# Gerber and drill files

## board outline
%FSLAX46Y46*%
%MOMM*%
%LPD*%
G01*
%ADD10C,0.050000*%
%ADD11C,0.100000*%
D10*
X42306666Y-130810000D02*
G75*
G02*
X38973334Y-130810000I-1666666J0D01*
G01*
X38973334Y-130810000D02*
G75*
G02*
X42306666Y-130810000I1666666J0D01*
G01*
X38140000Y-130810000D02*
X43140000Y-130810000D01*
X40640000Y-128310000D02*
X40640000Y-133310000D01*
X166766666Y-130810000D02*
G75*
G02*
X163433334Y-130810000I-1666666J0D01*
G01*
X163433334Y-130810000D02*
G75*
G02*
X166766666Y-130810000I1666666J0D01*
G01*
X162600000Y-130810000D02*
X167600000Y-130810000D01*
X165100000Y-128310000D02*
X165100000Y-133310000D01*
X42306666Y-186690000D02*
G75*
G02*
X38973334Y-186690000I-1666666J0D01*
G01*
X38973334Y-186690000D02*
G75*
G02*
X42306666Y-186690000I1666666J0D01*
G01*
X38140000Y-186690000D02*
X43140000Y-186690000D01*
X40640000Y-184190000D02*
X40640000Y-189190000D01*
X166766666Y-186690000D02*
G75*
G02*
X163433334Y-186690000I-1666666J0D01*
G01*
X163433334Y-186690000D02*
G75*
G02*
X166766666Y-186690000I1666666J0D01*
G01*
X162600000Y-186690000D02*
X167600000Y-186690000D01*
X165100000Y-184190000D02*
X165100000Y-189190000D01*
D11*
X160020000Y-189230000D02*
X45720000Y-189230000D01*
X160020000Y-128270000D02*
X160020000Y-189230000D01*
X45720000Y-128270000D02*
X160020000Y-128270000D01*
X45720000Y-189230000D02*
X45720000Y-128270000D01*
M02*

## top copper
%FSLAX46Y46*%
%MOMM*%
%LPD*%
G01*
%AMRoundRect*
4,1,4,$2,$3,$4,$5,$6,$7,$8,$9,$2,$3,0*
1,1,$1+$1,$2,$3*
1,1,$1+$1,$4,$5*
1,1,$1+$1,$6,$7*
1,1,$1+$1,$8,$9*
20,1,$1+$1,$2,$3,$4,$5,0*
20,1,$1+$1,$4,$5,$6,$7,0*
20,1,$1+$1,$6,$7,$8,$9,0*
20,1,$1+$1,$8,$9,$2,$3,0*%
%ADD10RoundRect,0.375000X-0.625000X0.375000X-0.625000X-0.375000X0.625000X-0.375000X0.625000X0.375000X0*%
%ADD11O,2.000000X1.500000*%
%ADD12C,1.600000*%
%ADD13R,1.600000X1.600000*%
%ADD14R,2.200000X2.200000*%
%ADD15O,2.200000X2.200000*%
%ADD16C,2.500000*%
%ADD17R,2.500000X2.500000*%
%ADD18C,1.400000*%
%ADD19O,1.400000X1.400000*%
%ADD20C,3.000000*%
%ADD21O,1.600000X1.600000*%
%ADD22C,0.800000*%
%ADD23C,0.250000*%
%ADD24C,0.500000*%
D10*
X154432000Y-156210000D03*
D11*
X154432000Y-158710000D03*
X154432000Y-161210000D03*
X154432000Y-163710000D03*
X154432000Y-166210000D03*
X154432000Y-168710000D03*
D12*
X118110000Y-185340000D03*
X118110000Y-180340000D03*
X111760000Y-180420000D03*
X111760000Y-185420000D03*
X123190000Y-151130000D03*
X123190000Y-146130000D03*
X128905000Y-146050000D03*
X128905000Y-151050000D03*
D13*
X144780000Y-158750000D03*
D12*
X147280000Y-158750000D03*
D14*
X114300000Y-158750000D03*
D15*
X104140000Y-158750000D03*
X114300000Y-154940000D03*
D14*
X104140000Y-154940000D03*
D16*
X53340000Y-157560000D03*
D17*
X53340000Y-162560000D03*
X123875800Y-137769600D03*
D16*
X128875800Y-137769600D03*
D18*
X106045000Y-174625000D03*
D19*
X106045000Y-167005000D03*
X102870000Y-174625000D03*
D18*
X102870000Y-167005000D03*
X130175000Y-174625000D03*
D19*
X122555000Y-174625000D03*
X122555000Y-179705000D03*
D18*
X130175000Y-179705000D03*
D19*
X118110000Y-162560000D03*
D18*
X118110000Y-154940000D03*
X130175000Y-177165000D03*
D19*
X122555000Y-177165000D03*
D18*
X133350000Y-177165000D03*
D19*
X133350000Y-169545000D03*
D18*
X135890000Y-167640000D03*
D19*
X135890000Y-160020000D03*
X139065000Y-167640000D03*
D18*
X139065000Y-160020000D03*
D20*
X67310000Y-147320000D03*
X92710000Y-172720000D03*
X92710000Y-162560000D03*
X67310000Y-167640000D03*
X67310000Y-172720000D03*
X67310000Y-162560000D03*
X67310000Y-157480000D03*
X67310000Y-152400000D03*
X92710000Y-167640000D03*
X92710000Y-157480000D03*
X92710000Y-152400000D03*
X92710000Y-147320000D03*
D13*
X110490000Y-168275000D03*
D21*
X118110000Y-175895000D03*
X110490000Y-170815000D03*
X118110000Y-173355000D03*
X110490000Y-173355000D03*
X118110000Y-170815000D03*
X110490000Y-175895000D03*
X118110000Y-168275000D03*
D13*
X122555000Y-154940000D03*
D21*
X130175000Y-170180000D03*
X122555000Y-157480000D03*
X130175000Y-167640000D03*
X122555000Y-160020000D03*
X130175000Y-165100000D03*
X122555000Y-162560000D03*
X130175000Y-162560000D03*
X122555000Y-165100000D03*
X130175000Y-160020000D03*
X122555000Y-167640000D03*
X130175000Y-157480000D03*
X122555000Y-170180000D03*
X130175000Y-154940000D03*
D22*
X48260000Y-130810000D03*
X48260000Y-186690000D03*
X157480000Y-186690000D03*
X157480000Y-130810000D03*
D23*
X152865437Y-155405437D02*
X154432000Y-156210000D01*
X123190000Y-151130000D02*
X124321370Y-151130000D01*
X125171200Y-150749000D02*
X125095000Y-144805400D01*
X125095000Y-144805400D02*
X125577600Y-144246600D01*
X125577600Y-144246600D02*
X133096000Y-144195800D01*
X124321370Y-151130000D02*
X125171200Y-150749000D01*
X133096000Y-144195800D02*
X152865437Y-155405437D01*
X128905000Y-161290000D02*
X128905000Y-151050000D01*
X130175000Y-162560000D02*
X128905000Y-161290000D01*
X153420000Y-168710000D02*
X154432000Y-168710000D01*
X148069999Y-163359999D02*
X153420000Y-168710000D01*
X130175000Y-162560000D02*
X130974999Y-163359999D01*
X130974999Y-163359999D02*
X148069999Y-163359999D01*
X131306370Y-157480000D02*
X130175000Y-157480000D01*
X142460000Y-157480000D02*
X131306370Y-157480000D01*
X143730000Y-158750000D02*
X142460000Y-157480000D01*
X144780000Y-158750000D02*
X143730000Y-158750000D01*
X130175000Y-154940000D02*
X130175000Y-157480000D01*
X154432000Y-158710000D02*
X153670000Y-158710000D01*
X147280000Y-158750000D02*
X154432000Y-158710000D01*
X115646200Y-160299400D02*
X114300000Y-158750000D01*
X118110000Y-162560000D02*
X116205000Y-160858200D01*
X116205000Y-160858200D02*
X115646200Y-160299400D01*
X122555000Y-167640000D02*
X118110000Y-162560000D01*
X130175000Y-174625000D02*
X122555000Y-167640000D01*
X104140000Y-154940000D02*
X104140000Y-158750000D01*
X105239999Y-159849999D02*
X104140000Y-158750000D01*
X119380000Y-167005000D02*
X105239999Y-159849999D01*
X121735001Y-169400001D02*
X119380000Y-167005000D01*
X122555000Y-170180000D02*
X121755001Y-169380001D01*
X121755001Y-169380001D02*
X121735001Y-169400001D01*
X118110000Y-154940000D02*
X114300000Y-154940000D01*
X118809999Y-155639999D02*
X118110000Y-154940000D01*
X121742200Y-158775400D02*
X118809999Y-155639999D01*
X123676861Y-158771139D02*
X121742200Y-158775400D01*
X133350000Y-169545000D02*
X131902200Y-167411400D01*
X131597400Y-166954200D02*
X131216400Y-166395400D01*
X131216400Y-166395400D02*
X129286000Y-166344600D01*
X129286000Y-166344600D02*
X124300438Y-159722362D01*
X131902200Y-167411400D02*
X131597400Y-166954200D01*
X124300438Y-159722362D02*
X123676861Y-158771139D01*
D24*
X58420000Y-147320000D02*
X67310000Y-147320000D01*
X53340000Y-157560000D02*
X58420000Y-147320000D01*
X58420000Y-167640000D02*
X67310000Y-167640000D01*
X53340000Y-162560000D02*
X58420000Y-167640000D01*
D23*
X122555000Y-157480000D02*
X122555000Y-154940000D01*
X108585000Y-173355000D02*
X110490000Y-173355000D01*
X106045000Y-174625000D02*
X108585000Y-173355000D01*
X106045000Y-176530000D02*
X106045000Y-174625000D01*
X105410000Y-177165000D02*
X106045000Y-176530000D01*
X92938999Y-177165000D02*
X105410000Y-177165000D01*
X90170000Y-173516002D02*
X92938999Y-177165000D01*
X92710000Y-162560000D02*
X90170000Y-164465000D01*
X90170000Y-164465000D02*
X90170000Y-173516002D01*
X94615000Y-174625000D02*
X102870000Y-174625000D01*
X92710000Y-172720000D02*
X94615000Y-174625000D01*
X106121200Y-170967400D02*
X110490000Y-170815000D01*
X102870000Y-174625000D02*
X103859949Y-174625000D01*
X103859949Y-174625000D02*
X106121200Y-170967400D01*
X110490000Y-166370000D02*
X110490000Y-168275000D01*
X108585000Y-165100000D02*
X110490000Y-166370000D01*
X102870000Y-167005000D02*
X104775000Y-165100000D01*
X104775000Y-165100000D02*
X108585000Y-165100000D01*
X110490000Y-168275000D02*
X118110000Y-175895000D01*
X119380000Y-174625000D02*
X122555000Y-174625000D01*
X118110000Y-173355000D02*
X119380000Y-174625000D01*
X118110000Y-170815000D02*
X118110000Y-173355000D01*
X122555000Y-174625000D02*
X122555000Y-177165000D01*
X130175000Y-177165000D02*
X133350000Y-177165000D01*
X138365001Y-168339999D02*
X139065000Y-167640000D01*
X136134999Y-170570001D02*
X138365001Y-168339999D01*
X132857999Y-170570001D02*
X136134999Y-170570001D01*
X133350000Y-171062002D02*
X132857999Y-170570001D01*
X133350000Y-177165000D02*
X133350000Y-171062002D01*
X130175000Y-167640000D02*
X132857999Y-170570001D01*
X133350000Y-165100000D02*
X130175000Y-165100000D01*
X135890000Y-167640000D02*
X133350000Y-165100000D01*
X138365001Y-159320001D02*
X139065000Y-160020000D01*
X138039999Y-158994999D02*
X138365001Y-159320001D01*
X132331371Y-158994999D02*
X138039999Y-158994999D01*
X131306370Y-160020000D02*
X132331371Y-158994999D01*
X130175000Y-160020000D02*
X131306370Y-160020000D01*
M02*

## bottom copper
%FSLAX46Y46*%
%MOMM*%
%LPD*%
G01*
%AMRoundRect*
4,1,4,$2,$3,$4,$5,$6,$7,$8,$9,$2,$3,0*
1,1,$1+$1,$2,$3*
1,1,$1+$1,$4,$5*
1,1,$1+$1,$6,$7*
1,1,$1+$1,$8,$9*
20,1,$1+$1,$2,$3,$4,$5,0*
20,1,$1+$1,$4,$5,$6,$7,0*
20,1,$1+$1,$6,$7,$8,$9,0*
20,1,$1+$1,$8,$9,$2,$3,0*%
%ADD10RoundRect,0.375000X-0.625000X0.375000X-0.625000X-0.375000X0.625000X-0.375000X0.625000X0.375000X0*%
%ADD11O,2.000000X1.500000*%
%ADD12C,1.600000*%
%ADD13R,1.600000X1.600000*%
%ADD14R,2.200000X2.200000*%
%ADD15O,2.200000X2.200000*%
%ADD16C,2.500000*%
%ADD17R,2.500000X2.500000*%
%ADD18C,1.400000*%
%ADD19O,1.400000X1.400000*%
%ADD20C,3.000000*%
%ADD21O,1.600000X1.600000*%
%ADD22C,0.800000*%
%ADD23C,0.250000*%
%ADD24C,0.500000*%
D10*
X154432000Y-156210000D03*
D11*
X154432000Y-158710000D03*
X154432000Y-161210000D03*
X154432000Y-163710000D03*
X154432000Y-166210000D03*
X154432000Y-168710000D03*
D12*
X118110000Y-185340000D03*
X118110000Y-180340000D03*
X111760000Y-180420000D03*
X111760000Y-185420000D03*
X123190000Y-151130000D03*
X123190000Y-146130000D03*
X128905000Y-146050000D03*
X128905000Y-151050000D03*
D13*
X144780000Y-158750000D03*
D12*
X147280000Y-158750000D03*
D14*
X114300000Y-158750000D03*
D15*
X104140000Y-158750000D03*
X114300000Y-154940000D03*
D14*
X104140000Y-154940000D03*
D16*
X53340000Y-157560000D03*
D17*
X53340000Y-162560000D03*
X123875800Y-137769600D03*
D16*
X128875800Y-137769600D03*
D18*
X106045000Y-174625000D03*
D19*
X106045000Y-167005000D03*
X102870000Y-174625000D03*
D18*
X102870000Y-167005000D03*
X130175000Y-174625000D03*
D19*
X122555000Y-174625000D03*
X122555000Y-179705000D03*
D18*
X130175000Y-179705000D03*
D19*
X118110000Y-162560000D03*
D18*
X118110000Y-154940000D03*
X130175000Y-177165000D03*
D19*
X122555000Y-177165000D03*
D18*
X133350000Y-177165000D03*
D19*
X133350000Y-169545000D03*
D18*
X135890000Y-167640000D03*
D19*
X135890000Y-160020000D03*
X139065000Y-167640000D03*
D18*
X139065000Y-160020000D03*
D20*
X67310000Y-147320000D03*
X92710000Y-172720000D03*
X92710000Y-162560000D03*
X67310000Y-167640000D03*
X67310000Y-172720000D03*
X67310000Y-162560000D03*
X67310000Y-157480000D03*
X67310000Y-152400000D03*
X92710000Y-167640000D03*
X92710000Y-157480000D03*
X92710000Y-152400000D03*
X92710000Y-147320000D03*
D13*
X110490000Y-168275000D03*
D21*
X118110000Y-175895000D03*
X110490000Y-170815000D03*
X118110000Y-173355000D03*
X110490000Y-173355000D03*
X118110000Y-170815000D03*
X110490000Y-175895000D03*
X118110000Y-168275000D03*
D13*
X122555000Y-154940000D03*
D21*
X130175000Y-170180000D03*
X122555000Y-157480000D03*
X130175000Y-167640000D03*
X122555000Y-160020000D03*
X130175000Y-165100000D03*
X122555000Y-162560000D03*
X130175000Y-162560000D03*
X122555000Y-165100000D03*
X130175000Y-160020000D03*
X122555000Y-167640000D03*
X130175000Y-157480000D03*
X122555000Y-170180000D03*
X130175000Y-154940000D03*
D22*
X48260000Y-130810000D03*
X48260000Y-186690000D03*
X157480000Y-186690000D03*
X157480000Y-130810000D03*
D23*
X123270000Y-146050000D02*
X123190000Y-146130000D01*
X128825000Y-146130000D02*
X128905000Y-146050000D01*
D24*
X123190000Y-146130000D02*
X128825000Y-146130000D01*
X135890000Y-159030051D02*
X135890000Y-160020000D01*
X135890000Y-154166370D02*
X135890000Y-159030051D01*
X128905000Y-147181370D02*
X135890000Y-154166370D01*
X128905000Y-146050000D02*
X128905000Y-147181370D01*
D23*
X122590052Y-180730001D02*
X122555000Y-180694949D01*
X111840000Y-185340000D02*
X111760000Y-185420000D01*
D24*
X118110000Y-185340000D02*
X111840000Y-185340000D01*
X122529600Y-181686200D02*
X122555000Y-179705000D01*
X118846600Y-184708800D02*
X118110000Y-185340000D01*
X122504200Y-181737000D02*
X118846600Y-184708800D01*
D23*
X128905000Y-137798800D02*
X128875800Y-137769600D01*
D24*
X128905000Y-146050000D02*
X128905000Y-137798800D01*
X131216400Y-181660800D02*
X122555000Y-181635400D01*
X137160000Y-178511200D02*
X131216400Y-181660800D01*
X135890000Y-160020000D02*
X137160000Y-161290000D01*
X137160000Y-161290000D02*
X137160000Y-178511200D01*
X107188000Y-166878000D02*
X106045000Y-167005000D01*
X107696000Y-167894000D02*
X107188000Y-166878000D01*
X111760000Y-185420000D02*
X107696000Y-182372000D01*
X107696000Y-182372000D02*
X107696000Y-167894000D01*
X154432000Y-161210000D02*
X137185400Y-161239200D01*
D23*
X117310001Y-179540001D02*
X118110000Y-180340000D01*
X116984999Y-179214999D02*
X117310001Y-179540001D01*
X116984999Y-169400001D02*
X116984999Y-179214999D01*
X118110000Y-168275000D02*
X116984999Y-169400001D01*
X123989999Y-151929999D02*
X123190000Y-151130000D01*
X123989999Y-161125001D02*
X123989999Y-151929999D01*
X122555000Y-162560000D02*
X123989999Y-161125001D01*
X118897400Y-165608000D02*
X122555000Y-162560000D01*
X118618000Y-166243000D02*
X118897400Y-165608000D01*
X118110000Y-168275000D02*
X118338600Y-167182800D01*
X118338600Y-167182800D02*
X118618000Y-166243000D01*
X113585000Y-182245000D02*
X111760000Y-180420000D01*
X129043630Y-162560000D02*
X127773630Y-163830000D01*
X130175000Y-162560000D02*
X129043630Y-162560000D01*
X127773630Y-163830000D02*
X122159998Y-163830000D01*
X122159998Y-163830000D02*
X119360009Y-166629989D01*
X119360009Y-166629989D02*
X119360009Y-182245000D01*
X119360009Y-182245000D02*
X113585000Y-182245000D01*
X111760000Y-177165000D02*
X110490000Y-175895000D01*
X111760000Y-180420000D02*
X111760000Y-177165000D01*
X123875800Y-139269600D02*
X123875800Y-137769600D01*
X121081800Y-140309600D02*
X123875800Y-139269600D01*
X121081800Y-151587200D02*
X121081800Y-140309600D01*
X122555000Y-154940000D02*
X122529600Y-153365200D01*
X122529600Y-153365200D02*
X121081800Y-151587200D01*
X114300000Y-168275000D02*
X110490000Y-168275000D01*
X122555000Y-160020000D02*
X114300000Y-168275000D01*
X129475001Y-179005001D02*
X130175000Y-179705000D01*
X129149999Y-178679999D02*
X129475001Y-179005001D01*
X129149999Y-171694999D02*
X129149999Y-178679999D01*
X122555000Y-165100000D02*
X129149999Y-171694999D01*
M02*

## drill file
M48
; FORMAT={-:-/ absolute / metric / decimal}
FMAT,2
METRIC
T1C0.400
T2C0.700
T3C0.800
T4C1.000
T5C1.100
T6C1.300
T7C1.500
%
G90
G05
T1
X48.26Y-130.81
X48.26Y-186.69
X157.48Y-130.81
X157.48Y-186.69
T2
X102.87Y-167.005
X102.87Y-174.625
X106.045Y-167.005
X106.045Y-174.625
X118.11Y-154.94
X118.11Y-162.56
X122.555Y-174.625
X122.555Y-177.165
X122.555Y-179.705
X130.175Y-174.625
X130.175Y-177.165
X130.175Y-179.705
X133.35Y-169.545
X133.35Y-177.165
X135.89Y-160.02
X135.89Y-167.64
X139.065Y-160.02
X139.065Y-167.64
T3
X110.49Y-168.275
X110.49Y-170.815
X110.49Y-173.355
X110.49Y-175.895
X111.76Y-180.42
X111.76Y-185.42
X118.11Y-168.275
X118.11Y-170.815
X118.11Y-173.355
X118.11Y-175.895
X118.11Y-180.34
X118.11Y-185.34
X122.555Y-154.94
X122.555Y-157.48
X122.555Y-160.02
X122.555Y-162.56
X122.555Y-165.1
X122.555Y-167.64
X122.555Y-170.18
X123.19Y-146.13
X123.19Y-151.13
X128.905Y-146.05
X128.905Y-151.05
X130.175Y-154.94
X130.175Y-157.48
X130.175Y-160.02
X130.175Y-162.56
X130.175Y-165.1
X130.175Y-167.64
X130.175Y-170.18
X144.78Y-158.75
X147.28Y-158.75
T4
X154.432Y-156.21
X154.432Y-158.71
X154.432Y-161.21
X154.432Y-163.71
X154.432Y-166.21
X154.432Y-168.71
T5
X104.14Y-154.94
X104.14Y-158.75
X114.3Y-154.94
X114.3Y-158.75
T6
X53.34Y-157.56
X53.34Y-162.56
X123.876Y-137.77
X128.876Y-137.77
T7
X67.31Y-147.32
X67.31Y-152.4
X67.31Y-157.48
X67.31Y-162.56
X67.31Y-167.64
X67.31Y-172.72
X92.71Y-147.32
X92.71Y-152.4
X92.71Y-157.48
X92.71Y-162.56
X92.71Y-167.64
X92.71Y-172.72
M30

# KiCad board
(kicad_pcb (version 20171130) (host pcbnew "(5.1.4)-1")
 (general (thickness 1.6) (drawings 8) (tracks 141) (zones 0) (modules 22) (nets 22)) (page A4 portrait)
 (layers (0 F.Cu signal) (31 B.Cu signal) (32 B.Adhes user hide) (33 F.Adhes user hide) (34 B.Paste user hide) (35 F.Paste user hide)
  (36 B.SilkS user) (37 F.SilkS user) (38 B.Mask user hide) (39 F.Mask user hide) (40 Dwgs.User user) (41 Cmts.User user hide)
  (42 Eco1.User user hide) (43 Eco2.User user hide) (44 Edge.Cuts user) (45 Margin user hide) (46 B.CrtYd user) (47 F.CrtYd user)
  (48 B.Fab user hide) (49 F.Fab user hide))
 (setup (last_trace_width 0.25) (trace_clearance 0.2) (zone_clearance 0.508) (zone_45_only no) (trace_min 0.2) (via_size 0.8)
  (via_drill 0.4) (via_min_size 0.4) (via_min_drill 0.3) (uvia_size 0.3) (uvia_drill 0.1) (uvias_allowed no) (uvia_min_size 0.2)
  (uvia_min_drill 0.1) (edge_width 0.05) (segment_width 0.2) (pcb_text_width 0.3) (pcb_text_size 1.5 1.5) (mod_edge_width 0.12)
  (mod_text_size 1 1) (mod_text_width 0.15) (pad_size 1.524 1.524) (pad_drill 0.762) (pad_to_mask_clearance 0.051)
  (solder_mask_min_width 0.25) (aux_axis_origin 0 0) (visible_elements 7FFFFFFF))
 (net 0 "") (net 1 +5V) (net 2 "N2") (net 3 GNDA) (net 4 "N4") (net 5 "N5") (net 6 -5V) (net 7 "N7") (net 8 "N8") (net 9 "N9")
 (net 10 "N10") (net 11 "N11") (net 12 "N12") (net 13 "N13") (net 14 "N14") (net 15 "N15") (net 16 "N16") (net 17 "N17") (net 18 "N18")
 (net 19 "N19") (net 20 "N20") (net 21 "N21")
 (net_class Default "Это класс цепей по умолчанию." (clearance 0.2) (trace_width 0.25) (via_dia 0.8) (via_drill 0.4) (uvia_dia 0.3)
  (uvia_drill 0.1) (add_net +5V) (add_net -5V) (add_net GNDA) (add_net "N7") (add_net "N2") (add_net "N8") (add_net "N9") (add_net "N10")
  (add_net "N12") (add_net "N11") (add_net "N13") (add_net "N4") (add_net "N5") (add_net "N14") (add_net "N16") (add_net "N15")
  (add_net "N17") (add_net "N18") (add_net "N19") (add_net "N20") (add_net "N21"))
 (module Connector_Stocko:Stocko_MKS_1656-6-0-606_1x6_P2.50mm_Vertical (layer F.Cu) (at 154.432 156.21 270)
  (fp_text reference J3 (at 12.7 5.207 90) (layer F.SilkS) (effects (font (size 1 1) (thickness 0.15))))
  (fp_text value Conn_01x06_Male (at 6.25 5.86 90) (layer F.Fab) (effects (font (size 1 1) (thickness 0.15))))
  (pad 1 thru_hole roundrect (at 0 0 270) (size 1.5 2) (drill 1) (layers *.Cu *.Mask) (roundrect_rratio 0.25) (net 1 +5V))
  (pad 2 thru_hole oval (at 2.5 0 270) (size 1.5 2) (drill 1) (layers *.Cu *.Mask) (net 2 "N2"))
  (pad 3 thru_hole oval (at 5 0 270) (size 1.5 2) (drill 1) (layers *.Cu *.Mask) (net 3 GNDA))
  (pad 4 thru_hole oval (at 7.5 0 270) (size 1.5 2) (drill 1) (layers *.Cu *.Mask) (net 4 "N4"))
  (pad 5 thru_hole oval (at 10 0 270) (size 1.5 2) (drill 1) (layers *.Cu *.Mask) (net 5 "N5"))
  (pad 6 thru_hole oval (at 12.5 0 270) (size 1.5 2) (drill 1) (layers *.Cu *.Mask) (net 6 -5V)))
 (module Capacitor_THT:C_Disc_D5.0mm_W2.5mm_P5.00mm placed (layer F.Cu) (at 118.11 180.34 270)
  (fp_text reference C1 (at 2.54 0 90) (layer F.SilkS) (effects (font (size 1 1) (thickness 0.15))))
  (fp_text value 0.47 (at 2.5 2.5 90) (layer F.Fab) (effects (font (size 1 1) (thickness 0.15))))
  (pad 2 thru_hole circle (at 5 0 270) (size 1.6 1.6) (drill 0.8) (layers *.Cu *.Mask) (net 3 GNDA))
  (pad 1 thru_hole circle (at 0 0 270) (size 1.6 1.6) (drill 0.8) (layers *.Cu *.Mask) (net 1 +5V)))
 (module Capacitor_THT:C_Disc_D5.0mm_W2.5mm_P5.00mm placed (layer F.Cu) (at 111.76 185.42 90)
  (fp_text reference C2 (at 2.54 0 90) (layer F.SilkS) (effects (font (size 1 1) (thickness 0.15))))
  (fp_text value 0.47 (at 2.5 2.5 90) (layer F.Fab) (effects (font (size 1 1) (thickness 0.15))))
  (pad 2 thru_hole circle (at 5 0 90) (size 1.6 1.6) (drill 0.8) (layers *.Cu *.Mask) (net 6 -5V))
  (pad 1 thru_hole circle (at 0 0 90) (size 1.6 1.6) (drill 0.8) (layers *.Cu *.Mask) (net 3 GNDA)))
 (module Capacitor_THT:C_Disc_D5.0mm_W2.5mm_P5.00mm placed (layer F.Cu) (at 123.19 151.13 90)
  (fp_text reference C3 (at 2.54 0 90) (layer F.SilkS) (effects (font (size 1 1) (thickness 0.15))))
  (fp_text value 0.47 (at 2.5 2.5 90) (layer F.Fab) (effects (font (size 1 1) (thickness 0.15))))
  (pad 1 thru_hole circle (at 0 0 90) (size 1.6 1.6) (drill 0.8) (layers *.Cu *.Mask) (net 1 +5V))
  (pad 2 thru_hole circle (at 5 0 90) (size 1.6 1.6) (drill 0.8) (layers *.Cu *.Mask) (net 3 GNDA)))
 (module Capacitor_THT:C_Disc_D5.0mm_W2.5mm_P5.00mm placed (layer F.Cu) (at 128.905 146.05 270)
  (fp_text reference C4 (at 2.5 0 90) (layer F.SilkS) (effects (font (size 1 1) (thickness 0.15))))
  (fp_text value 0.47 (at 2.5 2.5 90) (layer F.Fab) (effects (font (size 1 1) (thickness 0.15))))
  (pad 1 thru_hole circle (at 0 0 270) (size 1.6 1.6) (drill 0.8) (layers *.Cu *.Mask) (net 3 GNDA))
  (pad 2 thru_hole circle (at 5 0 270) (size 1.6 1.6) (drill 0.8) (layers *.Cu *.Mask) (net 6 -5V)))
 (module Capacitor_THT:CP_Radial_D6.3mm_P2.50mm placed (layer F.Cu) (at 144.78 158.75)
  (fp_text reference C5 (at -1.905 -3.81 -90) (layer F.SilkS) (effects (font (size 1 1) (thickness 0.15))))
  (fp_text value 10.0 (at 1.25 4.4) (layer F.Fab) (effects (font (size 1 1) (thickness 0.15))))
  (pad 1 thru_hole rect (at 0 0) (size 1.6 1.6) (drill 0.8) (layers *.Cu *.Mask) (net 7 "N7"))
  (pad 2 thru_hole circle (at 2.5 0) (size 1.6 1.6) (drill 0.8) (layers *.Cu *.Mask) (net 2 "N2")))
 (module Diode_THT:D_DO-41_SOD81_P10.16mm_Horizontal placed (layer F.Cu) (at 114.3 158.75 180)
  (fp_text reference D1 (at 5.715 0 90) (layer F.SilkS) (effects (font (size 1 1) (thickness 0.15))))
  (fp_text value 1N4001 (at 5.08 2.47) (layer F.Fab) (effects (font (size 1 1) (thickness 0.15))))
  (pad 1 thru_hole rect (at 0 0 180) (size 2.2 2.2) (drill 1.1) (layers *.Cu *.Mask) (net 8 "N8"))
  (pad 2 thru_hole oval (at 10.16 0 180) (size 2.2 2.2) (drill 1.1) (layers *.Cu *.Mask) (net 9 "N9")))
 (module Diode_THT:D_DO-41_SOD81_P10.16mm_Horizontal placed (layer F.Cu) (at 104.14 154.94)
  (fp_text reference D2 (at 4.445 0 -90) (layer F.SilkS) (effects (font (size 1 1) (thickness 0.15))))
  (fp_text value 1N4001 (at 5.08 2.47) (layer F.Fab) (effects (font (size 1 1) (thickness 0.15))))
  (pad 2 thru_hole oval (at 10.16 0) (size 2.2 2.2) (drill 1.1) (layers *.Cu *.Mask) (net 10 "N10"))
  (pad 1 thru_hole rect (at 0 0) (size 2.2 2.2) (drill 1.1) (layers *.Cu *.Mask) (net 9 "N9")))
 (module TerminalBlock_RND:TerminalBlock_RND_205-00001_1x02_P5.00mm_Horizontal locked (layer F.Cu) (at 53.34 162.56 90)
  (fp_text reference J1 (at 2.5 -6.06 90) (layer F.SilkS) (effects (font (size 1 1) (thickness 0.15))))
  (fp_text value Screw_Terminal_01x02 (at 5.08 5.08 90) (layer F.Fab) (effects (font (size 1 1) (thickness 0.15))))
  (pad 2 thru_hole circle (at 5 0 90) (size 2.5 2.5) (drill 1.3) (layers *.Cu *.Mask) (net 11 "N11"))
  (pad 1 thru_hole rect (at 0 0 90) (size 2.5 2.5) (drill 1.3) (layers *.Cu *.Mask) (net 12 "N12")))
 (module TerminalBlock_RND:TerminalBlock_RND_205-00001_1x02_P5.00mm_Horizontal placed (layer F.Cu) (at 123.8758 137.7696)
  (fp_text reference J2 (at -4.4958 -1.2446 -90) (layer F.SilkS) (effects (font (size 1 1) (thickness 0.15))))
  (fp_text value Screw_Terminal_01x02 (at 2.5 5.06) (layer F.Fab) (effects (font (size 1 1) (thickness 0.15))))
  (pad 1 thru_hole rect (at 0 0) (size 2.5 2.5) (drill 1.3) (layers *.Cu *.Mask) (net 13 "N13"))
  (pad 2 thru_hole circle (at 5 0) (size 2.5 2.5) (drill 1.3) (layers *.Cu *.Mask) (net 3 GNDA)))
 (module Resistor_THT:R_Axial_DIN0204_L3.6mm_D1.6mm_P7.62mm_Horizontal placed (layer F.Cu) (at 106.045 174.625 90)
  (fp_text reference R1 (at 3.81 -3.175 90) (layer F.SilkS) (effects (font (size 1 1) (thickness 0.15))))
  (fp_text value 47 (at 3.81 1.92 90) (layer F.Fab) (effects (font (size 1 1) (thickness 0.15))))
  (pad 1 thru_hole circle (at 0 0 90) (size 1.4 1.4) (drill 0.7) (layers *.Cu *.Mask) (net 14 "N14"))
  (pad 2 thru_hole oval (at 7.62 0 90) (size 1.4 1.4) (drill 0.7) (layers *.Cu *.Mask) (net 3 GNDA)))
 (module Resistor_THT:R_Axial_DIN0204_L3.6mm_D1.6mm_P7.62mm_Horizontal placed (layer F.Cu) (at 102.87 167.005 270)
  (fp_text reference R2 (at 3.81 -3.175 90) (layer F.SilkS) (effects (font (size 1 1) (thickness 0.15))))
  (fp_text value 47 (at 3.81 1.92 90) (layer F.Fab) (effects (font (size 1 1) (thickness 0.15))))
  (pad 2 thru_hole oval (at 7.62 0 270) (size 1.4 1.4) (drill 0.7) (layers *.Cu *.Mask) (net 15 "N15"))
  (pad 1 thru_hole circle (at 0 0 270) (size 1.4 1.4) (drill 0.7) (layers *.Cu *.Mask) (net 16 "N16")))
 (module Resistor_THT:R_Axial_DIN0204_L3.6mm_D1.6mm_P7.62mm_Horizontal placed (layer F.Cu) (at 130.175 174.625 180)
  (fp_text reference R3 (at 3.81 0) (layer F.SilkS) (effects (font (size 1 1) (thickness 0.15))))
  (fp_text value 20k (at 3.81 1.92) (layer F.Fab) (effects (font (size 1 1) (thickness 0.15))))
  (pad 1 thru_hole circle (at 0 0 180) (size 1.4 1.4) (drill 0.7) (layers *.Cu *.Mask) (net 8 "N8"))
  (pad 2 thru_hole oval (at 7.62 0 180) (size 1.4 1.4) (drill 0.7) (layers *.Cu *.Mask) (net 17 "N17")))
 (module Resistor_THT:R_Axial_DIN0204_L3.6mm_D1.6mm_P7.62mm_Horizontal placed (layer F.Cu) (at 130.175 179.705 180)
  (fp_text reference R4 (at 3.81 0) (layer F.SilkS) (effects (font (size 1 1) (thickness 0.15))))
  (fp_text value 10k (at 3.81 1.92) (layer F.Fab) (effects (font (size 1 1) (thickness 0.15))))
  (pad 2 thru_hole oval (at 7.62 0 180) (size 1.4 1.4) (drill 0.7) (layers *.Cu *.Mask) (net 3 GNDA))
  (pad 1 thru_hole circle (at 0 0 180) (size 1.4 1.4) (drill 0.7) (layers *.Cu *.Mask) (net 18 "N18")))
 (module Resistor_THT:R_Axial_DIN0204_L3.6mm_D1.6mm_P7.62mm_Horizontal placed (layer F.Cu) (at 118.11 154.94 270)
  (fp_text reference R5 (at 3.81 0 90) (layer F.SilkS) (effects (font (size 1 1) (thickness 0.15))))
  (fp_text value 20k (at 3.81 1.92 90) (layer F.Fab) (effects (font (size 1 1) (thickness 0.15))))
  (pad 2 thru_hole oval (at 7.62 0 270) (size 1.4 1.4) (drill 0.7) (layers *.Cu *.Mask) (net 8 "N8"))
  (pad 1 thru_hole circle (at 0 0 270) (size 1.4 1.4) (drill 0.7) (layers *.Cu *.Mask) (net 10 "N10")))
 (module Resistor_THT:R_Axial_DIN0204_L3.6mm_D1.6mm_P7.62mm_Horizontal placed (layer F.Cu) (at 130.175 177.165 180)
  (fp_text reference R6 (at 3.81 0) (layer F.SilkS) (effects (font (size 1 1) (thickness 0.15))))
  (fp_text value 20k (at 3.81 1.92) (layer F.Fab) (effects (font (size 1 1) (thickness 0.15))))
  (pad 1 thru_hole circle (at 0 0 180) (size 1.4 1.4) (drill 0.7) (layers *.Cu *.Mask) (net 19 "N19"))
  (pad 2 thru_hole oval (at 7.62 0 180) (size 1.4 1.4) (drill 0.7) (layers *.Cu *.Mask) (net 17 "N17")))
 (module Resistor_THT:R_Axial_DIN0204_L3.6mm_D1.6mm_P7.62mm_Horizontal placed (layer F.Cu) (at 133.35 177.165 90)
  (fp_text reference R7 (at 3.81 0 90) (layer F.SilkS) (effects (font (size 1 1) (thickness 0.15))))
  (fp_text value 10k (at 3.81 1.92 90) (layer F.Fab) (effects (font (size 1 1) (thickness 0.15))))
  (pad 1 thru_hole circle (at 0 0 90) (size 1.4 1.4) (drill 0.7) (layers *.Cu *.Mask) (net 19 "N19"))
  (pad 2 thru_hole oval (at 7.62 0 90) (size 1.4 1.4) (drill 0.7) (layers *.Cu *.Mask) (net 10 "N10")))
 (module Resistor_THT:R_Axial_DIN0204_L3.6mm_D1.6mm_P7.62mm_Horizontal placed (layer F.Cu) (at 135.89 167.64 90)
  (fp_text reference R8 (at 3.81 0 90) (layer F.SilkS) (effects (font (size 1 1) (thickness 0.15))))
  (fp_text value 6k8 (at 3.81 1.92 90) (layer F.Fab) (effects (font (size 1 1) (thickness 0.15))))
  (pad 1 thru_hole circle (at 0 0 90) (size 1.4 1.4) (drill 0.7) (layers *.Cu *.Mask) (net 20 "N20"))
  (pad 2 thru_hole oval (at 7.62 0 90) (size 1.4 1.4) (drill 0.7) (layers *.Cu *.Mask) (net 3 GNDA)))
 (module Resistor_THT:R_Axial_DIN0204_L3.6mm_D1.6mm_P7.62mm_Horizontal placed (layer F.Cu) (at 139.065 160.02 270)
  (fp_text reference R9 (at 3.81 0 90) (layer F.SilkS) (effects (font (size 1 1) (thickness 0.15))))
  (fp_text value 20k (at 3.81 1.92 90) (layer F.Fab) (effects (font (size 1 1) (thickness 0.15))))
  (pad 2 thru_hole oval (at 7.62 0 270) (size 1.4 1.4) (drill 0.7) (layers *.Cu *.Mask) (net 19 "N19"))
  (pad 1 thru_hole circle (at 0 0 270) (size 1.4 1.4) (drill 0.7) (layers *.Cu *.Mask) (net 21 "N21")))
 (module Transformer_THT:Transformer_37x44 (layer F.Cu) (at 67.31 167.64 90)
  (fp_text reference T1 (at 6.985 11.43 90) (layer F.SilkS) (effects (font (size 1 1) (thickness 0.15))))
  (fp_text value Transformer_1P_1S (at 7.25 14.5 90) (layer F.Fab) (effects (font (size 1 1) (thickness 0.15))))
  (pad 2 thru_hole circle (at 20.32 0 90) (size 3 3) (drill 1.5) (layers *.Cu *.Mask) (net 11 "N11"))
  (pad 4 thru_hole circle (at -5.08 25.4 90) (size 3 3) (drill 1.5) (layers *.Cu *.Mask) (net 15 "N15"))
  (pad 3 thru_hole circle (at 5.08 25.4 90) (size 3 3) (drill 1.5) (layers *.Cu *.Mask) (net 14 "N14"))
  (pad 1 thru_hole circle (at 0 0 90) (size 3 3) (drill 1.5) (layers *.Cu *.Mask) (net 12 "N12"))
  (pad "" thru_hole circle (at -5.08 0 90) (size 3 3) (drill 1.5) (layers *.Cu *.Mask))
  (pad "" thru_hole circle (at 5.08 0 90) (size 3 3) (drill 1.5) (layers *.Cu *.Mask))
  (pad "" thru_hole circle (at 10.16 0 90) (size 3 3) (drill 1.5) (layers *.Cu *.Mask))
  (pad "" thru_hole circle (at 15.24 0 90) (size 3 3) (drill 1.5) (layers *.Cu *.Mask))
  (pad "" thru_hole circle (at 0 25.4 90) (size 3 3) (drill 1.5) (layers *.Cu *.Mask))
  (pad "" thru_hole circle (at 10.16 25.4 90) (size 3 3) (drill 1.5) (layers *.Cu *.Mask))
  (pad "" thru_hole circle (at 15.24 25.4 90) (size 3 3) (drill 1.5) (layers *.Cu *.Mask))
  (pad "" thru_hole circle (at 20.32 25.4 90) (size 3 3) (drill 1.5) (layers *.Cu *.Mask)))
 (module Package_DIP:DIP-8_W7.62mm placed (layer F.Cu) (at 110.49 168.275)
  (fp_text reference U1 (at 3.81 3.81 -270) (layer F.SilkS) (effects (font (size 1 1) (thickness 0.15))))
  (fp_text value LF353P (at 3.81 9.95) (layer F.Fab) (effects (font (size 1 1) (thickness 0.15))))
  (pad 1 thru_hole rect (at 0 0) (size 1.6 1.6) (drill 0.8) (layers *.Cu *.Mask) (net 16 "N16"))
  (pad 5 thru_hole oval (at 7.62 7.62) (size 1.6 1.6) (drill 0.8) (layers *.Cu *.Mask) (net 16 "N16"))
  (pad 2 thru_hole oval (at 0 2.54) (size 1.6 1.6) (drill 0.8) (layers *.Cu *.Mask) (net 15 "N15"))
  (pad 6 thru_hole oval (at 7.62 5.08) (size 1.6 1.6) (drill 0.8) (layers *.Cu *.Mask) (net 17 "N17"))
  (pad 3 thru_hole oval (at 0 5.08) (size 1.6 1.6) (drill 0.8) (layers *.Cu *.Mask) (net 14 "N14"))
  (pad 7 thru_hole oval (at 7.62 2.54) (size 1.6 1.6) (drill 0.8) (layers *.Cu *.Mask) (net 17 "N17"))
  (pad 4 thru_hole oval (at 0 7.62) (size 1.6 1.6) (drill 0.8) (layers *.Cu *.Mask) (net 6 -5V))
  (pad 8 thru_hole oval (at 7.62 0) (size 1.6 1.6) (drill 0.8) (layers *.Cu *.Mask) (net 1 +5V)))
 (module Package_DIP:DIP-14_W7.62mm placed (layer F.Cu) (at 122.555 154.94)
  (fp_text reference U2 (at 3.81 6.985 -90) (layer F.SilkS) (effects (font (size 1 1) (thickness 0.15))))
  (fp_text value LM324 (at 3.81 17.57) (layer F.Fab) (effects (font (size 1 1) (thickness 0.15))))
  (pad 1 thru_hole rect (at 0 0) (size 1.6 1.6) (drill 0.8) (layers *.Cu *.Mask) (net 13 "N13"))
  (pad 8 thru_hole oval (at 7.62 15.24) (size 1.6 1.6) (drill 0.8) (layers *.Cu *.Mask) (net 21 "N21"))
  (pad 2 thru_hole oval (at 0 2.54) (size 1.6 1.6) (drill 0.8) (layers *.Cu *.Mask) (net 13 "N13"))
  (pad 9 thru_hole oval (at 7.62 12.7) (size 1.6 1.6) (drill 0.8) (layers *.Cu *.Mask) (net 19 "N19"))
  (pad 3 thru_hole oval (at 0 5.08) (size 1.6 1.6) (drill 0.8) (layers *.Cu *.Mask) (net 16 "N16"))
  (pad 10 thru_hole oval (at 7.62 10.16) (size 1.6 1.6) (drill 0.8) (layers *.Cu *.Mask) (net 20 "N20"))
  (pad 4 thru_hole oval (at 0 7.62) (size 1.6 1.6) (drill 0.8) (layers *.Cu *.Mask) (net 1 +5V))
  (pad 11 thru_hole oval (at 7.62 7.62) (size 1.6 1.6) (drill 0.8) (layers *.Cu *.Mask) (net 6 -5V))
  (pad 5 thru_hole oval (at 0 10.16) (size 1.6 1.6) (drill 0.8) (layers *.Cu *.Mask) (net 18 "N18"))
  (pad 12 thru_hole oval (at 7.62 5.08) (size 1.6 1.6) (drill 0.8) (layers *.Cu *.Mask) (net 21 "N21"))
  (pad 6 thru_hole oval (at 0 12.7) (size 1.6 1.6) (drill 0.8) (layers *.Cu *.Mask) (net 8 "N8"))
  (pad 13 thru_hole oval (at 7.62 2.54) (size 1.6 1.6) (drill 0.8) (layers *.Cu *.Mask) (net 7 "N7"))
  (pad 7 thru_hole oval (at 0 15.24) (size 1.6 1.6) (drill 0.8) (layers *.Cu *.Mask) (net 9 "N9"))
  (pad 14 thru_hole oval (at 7.62 0) (size 1.6 1.6) (drill 0.8) (layers *.Cu *.Mask) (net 7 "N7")))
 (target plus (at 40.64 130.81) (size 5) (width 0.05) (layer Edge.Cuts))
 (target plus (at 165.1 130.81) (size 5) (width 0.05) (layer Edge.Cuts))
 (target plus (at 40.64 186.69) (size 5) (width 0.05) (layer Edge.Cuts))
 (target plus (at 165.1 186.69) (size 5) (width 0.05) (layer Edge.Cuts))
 (gr_line (start 160.02 189.23) (end 45.72 189.23) (layer Edge.Cuts) (width 0.1))
 (gr_line (start 160.02 128.27) (end 160.02 189.23) (layer Edge.Cuts) (width 0.1))
 (gr_line (start 45.72 128.27) (end 160.02 128.27) (layer Edge.Cuts) (width 0.1))
 (gr_line (start 45.72 189.23) (end 45.72 128.27) (layer Edge.Cuts) (width 0.1))
 (via (at 48.26 130.81) (size 0.8) (drill 0.4) (layers F.Cu B.Cu) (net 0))
 (via (at 48.26 186.69) (size 0.8) (drill 0.4) (layers F.Cu B.Cu) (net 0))
 (via (at 157.48 186.69) (size 0.8) (drill 0.4) (layers F.Cu B.Cu) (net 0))
 (via (at 157.48 130.81) (size 0.8) (drill 0.4) (layers F.Cu B.Cu) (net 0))
 (segment (start 123.27 146.05) (end 123.19 146.13) (width 0.25) (layer B.Cu) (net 3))
 (segment (start 128.825 146.13) (end 128.905 146.05) (width 0.25) (layer B.Cu) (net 3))
 (segment (start 123.19 146.13) (end 128.825 146.13) (width 0.5) (layer B.Cu) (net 3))
 (segment (start 135.89 159.030051) (end 135.89 160.02) (width 0.5) (layer B.Cu) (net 3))
 (segment (start 135.89 154.16637) (end 135.89 159.030051) (width 0.5) (layer B.Cu) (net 3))
 (segment (start 128.905 147.18137) (end 135.89 154.16637) (width 0.5) (layer B.Cu) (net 3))
 (segment (start 128.905 146.05) (end 128.905 147.18137) (width 0.5) (layer B.Cu) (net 3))
 (segment (start 122.590052 180.730001) (end 122.555 180.694949) (width 0.25) (layer B.Cu) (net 3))
 (segment (start 111.84 185.34) (end 111.76 185.42) (width 0.25) (layer B.Cu) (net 3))
 (segment (start 118.11 185.34) (end 111.84 185.34) (width 0.5) (layer B.Cu) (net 3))
 (segment (start 122.5296 181.6862) (end 122.555 179.705) (width 0.5) (layer B.Cu) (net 3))
 (segment (start 118.8466 184.7088) (end 118.11 185.34) (width 0.5) (layer B.Cu) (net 3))
 (segment (start 122.5042 181.737) (end 118.8466 184.7088) (width 0.5) (layer B.Cu) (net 3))
 (segment (start 128.905 137.7988) (end 128.8758 137.7696) (width 0.25) (layer B.Cu) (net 3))
 (segment (start 128.905 146.05) (end 128.905 137.7988) (width 0.5) (layer B.Cu) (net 3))
 (segment (start 131.2164 181.6608) (end 122.555 181.6354) (width 0.5) (layer B.Cu) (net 3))
 (segment (start 137.16 178.5112) (end 131.2164 181.6608) (width 0.5) (layer B.Cu) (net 3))
 (segment (start 135.89 160.02) (end 137.16 161.29) (width 0.5) (layer B.Cu) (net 3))
 (segment (start 137.16 161.29) (end 137.16 178.5112) (width 0.5) (layer B.Cu) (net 3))
 (segment (start 107.188 166.878) (end 106.045 167.005) (width 0.5) (layer B.Cu) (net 3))
 (segment (start 107.696 167.894) (end 107.188 166.878) (width 0.5) (layer B.Cu) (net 3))
 (segment (start 111.76 185.42) (end 107.696 182.372) (width 0.5) (layer B.Cu) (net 3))
 (segment (start 107.696 182.372) (end 107.696 167.894) (width 0.5) (layer B.Cu) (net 3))
 (segment (start 154.432 161.21) (end 137.1854 161.2392) (width 0.5) (layer B.Cu) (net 3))
 (segment (start 117.310001 179.540001) (end 118.11 180.34) (width 0.25) (layer B.Cu) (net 1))
 (segment (start 116.984999 179.214999) (end 117.310001 179.540001) (width 0.25) (layer B.Cu) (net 1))
 (segment (start 116.984999 169.400001) (end 116.984999 179.214999) (width 0.25) (layer B.Cu) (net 1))
 (segment (start 118.11 168.275) (end 116.984999 169.400001) (width 0.25) (layer B.Cu) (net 1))
 (segment (start 123.989999 151.929999) (end 123.19 151.13) (width 0.25) (layer B.Cu) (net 1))
 (segment (start 123.989999 161.125001) (end 123.989999 151.929999) (width 0.25) (layer B.Cu) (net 1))
 (segment (start 122.555 162.56) (end 123.989999 161.125001) (width 0.25) (layer B.Cu) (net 1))
 (segment (start 118.8974 165.608) (end 122.555 162.56) (width 0.25) (layer B.Cu) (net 1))
 (segment (start 118.618 166.243) (end 118.8974 165.608) (width 0.25) (layer B.Cu) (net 1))
 (segment (start 118.11 168.275) (end 118.3386 167.1828) (width 0.25) (layer B.Cu) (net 1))
 (segment (start 118.3386 167.1828) (end 118.618 166.243) (width 0.25) (layer B.Cu) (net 1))
 (segment (start 152.865437 155.405437) (end 154.432 156.21) (width 0.25) (layer F.Cu) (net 1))
 (segment (start 123.19 151.13) (end 124.32137 151.13) (width 0.25) (layer F.Cu) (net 1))
 (segment (start 125.1712 150.749) (end 125.095 144.8054) (width 0.25) (layer F.Cu) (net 1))
 (segment (start 125.095 144.8054) (end 125.5776 144.2466) (width 0.25) (layer F.Cu) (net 1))
 (segment (start 125.5776 144.2466) (end 133.096 144.1958) (width 0.25) (layer F.Cu) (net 1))
 (segment (start 124.32137 151.13) (end 125.1712 150.749) (width 0.25) (layer F.Cu) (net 1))
 (segment (start 133.096 144.1958) (end 152.865437 155.405437) (width 0.25) (layer F.Cu) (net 1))
 (segment (start 113.585 182.245) (end 111.76 180.42) (width 0.25) (layer B.Cu) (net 6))
 (segment (start 129.04363 162.56) (end 127.77363 163.83) (width 0.25) (layer B.Cu) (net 6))
 (segment (start 130.175 162.56) (end 129.04363 162.56) (width 0.25) (layer B.Cu) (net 6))
 (segment (start 127.77363 163.83) (end 122.159998 163.83) (width 0.25) (layer B.Cu) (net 6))
 (segment (start 122.159998 163.83) (end 119.360009 166.629989) (width 0.25) (layer B.Cu) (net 6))
 (segment (start 119.360009 166.629989) (end 119.360009 182.245) (width 0.25) (layer B.Cu) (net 6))
 (segment (start 119.360009 182.245) (end 113.585 182.245) (width 0.25) (layer B.Cu) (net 6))
 (segment (start 111.76 177.165) (end 110.49 175.895) (width 0.25) (layer B.Cu) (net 6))
 (segment (start 111.76 180.42) (end 111.76 177.165) (width 0.25) (layer B.Cu) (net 6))
 (segment (start 128.905 161.29) (end 128.905 151.05) (width 0.25) (layer F.Cu) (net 6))
 (segment (start 130.175 162.56) (end 128.905 161.29) (width 0.25) (layer F.Cu) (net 6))
 (segment (start 153.42 168.71) (end 154.432 168.71) (width 0.25) (layer F.Cu) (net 6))
 (segment (start 148.069999 163.359999) (end 153.42 168.71) (width 0.25) (layer F.Cu) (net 6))
 (segment (start 130.175 162.56) (end 130.974999 163.359999) (width 0.25) (layer F.Cu) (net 6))
 (segment (start 130.974999 163.359999) (end 148.069999 163.359999) (width 0.25) (layer F.Cu) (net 6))
 (segment (start 131.30637 157.48) (end 130.175 157.48) (width 0.25) (layer F.Cu) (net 7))
 (segment (start 142.46 157.48) (end 131.30637 157.48) (width 0.25) (layer F.Cu) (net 7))
 (segment (start 143.73 158.75) (end 142.46 157.48) (width 0.25) (layer F.Cu) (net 7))
 (segment (start 144.78 158.75) (end 143.73 158.75) (width 0.25) (layer F.Cu) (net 7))
 (segment (start 130.175 154.94) (end 130.175 157.48) (width 0.25) (layer F.Cu) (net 7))
 (segment (start 154.432 158.71) (end 153.67 158.71) (width 0.25) (layer F.Cu) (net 2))
 (segment (start 147.28 158.75) (end 154.432 158.71) (width 0.25) (layer F.Cu) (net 2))
 (segment (start 115.6462 160.2994) (end 114.3 158.75) (width 0.25) (layer F.Cu) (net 8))
 (segment (start 118.11 162.56) (end 116.205 160.8582) (width 0.25) (layer F.Cu) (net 8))
 (segment (start 116.205 160.8582) (end 115.6462 160.2994) (width 0.25) (layer F.Cu) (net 8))
 (segment (start 122.555 167.64) (end 118.11 162.56) (width 0.25) (layer F.Cu) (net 8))
 (segment (start 130.175 174.625) (end 122.555 167.64) (width 0.25) (layer F.Cu) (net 8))
 (segment (start 104.14 154.94) (end 104.14 158.75) (width 0.25) (layer F.Cu) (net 9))
 (segment (start 105.239999 159.849999) (end 104.14 158.75) (width 0.25) (layer F.Cu) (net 9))
 (segment (start 119.38 167.005) (end 105.239999 159.849999) (width 0.25) (layer F.Cu) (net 9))
 (segment (start 121.735001 169.400001) (end 119.38 167.005) (width 0.25) (layer F.Cu) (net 9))
 (segment (start 122.555 170.18) (end 121.755001 169.380001) (width 0.25) (layer F.Cu) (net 9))
 (segment (start 121.755001 169.380001) (end 121.735001 169.400001) (width 0.25) (layer F.Cu) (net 9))
 (segment (start 118.11 154.94) (end 114.3 154.94) (width 0.25) (layer F.Cu) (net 10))
 (segment (start 118.809999 155.639999) (end 118.11 154.94) (width 0.25) (layer F.Cu) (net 10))
 (segment (start 121.7422 158.7754) (end 118.809999 155.639999) (width 0.25) (layer F.Cu) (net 10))
 (segment (start 123.676861 158.771139) (end 121.7422 158.7754) (width 0.25) (layer F.Cu) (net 10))
 (segment (start 133.35 169.545) (end 131.9022 167.4114) (width 0.25) (layer F.Cu) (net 10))
 (segment (start 131.5974 166.9542) (end 131.2164 166.3954) (width 0.25) (layer F.Cu) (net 10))
 (segment (start 131.2164 166.3954) (end 129.286 166.3446) (width 0.25) (layer F.Cu) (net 10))
 (segment (start 129.286 166.3446) (end 124.300438 159.722362) (width 0.25) (layer F.Cu) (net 10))
 (segment (start 131.9022 167.4114) (end 131.5974 166.9542) (width 0.25) (layer F.Cu) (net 10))
 (segment (start 124.300438 159.722362) (end 123.676861 158.771139) (width 0.25) (layer F.Cu) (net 10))
 (segment (start 58.42 147.32) (end 67.31 147.32) (width 0.5) (layer F.Cu) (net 11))
 (segment (start 53.34 157.56) (end 58.42 147.32) (width 0.5) (layer F.Cu) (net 11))
 (segment (start 58.42 167.64) (end 67.31 167.64) (width 0.5) (layer F.Cu) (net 12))
 (segment (start 53.34 162.56) (end 58.42 167.64) (width 0.5) (layer F.Cu) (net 12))
 (segment (start 122.555 157.48) (end 122.555 154.94) (width 0.25) (layer F.Cu) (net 13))
 (segment (start 123.8758 139.2696) (end 123.8758 137.7696) (width 0.25) (layer B.Cu) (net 13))
 (segment (start 121.0818 140.3096) (end 123.8758 139.2696) (width 0.25) (layer B.Cu) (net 13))
 (segment (start 121.0818 151.5872) (end 121.0818 140.3096) (width 0.25) (layer B.Cu) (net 13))
 (segment (start 122.555 154.94) (end 122.5296 153.3652) (width 0.25) (layer B.Cu) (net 13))
 (segment (start 122.5296 153.3652) (end 121.0818 151.5872) (width 0.25) (layer B.Cu) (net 13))
 (segment (start 108.585 173.355) (end 110.49 173.355) (width 0.25) (layer F.Cu) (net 14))
 (segment (start 106.045 174.625) (end 108.585 173.355) (width 0.25) (layer F.Cu) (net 14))
 (segment (start 106.045 176.53) (end 106.045 174.625) (width 0.25) (layer F.Cu) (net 14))
 (segment (start 105.41 177.165) (end 106.045 176.53) (width 0.25) (layer F.Cu) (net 14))
 (segment (start 92.938999 177.165) (end 105.41 177.165) (width 0.25) (layer F.Cu) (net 14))
 (segment (start 90.17 173.516002) (end 92.938999 177.165) (width 0.25) (layer F.Cu) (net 14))
 (segment (start 92.71 162.56) (end 90.17 164.465) (width 0.25) (layer F.Cu) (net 14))
 (segment (start 90.17 164.465) (end 90.17 173.516002) (width 0.25) (layer F.Cu) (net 14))
 (segment (start 94.615 174.625) (end 102.87 174.625) (width 0.25) (layer F.Cu) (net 15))
 (segment (start 92.71 172.72) (end 94.615 174.625) (width 0.25) (layer F.Cu) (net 15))
 (segment (start 106.1212 170.9674) (end 110.49 170.815) (width 0.25) (layer F.Cu) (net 15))
 (segment (start 102.87 174.625) (end 103.859949 174.625) (width 0.25) (layer F.Cu) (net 15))
 (segment (start 103.859949 174.625) (end 106.1212 170.9674) (width 0.25) (layer F.Cu) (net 15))
 (segment (start 110.49 166.37) (end 110.49 168.275) (width 0.25) (layer F.Cu) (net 16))
 (segment (start 108.585 165.1) (end 110.49 166.37) (width 0.25) (layer F.Cu) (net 16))
 (segment (start 102.87 167.005) (end 104.775 165.1) (width 0.25) (layer F.Cu) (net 16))
 (segment (start 104.775 165.1) (end 108.585 165.1) (width 0.25) (layer F.Cu) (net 16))
 (segment (start 110.49 168.275) (end 118.11 175.895) (width 0.25) (layer F.Cu) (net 16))
 (segment (start 114.3 168.275) (end 110.49 168.275) (width 0.25) (layer B.Cu) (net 16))
 (segment (start 122.555 160.02) (end 114.3 168.275) (width 0.25) (layer B.Cu) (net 16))
 (segment (start 119.38 174.625) (end 122.555 174.625) (width 0.25) (layer F.Cu) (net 17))
 (segment (start 118.11 173.355) (end 119.38 174.625) (width 0.25) (layer F.Cu) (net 17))
 (segment (start 118.11 170.815) (end 118.11 173.355) (width 0.25) (layer F.Cu) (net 17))
 (segment (start 122.555 174.625) (end 122.555 177.165) (width 0.25) (layer F.Cu) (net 17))
 (segment (start 129.475001 179.005001) (end 130.175 179.705) (width 0.25) (layer B.Cu) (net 18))
 (segment (start 129.149999 178.679999) (end 129.475001 179.005001) (width 0.25) (layer B.Cu) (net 18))
 (segment (start 129.149999 171.694999) (end 129.149999 178.679999) (width 0.25) (layer B.Cu) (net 18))
 (segment (start 122.555 165.1) (end 129.149999 171.694999) (width 0.25) (layer B.Cu) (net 18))
 (segment (start 130.175 177.165) (end 133.35 177.165) (width 0.25) (layer F.Cu) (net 19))
 (segment (start 138.365001 168.339999) (end 139.065 167.64) (width 0.25) (layer F.Cu) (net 19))
 (segment (start 136.134999 170.570001) (end 138.365001 168.339999) (width 0.25) (layer F.Cu) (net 19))
 (segment (start 132.857999 170.570001) (end 136.134999 170.570001) (width 0.25) (layer F.Cu) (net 19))
 (segment (start 133.35 171.062002) (end 132.857999 170.570001) (width 0.25) (layer F.Cu) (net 19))
 (segment (start 133.35 177.165) (end 133.35 171.062002) (width 0.25) (layer F.Cu) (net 19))
 (segment (start 130.175 167.64) (end 132.857999 170.570001) (width 0.25) (layer F.Cu) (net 19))
 (segment (start 133.35 165.1) (end 130.175 165.1) (width 0.25) (layer F.Cu) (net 20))
 (segment (start 135.89 167.64) (end 133.35 165.1) (width 0.25) (layer F.Cu) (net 20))
 (segment (start 138.365001 159.320001) (end 139.065 160.02) (width 0.25) (layer F.Cu) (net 21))
 (segment (start 138.039999 158.994999) (end 138.365001 159.320001) (width 0.25) (layer F.Cu) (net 21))
 (segment (start 132.331371 158.994999) (end 138.039999 158.994999) (width 0.25) (layer F.Cu) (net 21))
 (segment (start 131.30637 160.02) (end 132.331371 158.994999) (width 0.25) (layer F.Cu) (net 21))
 (segment (start 130.175 160.02) (end 131.30637 160.02) (width 0.25) (layer F.Cu) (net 21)))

